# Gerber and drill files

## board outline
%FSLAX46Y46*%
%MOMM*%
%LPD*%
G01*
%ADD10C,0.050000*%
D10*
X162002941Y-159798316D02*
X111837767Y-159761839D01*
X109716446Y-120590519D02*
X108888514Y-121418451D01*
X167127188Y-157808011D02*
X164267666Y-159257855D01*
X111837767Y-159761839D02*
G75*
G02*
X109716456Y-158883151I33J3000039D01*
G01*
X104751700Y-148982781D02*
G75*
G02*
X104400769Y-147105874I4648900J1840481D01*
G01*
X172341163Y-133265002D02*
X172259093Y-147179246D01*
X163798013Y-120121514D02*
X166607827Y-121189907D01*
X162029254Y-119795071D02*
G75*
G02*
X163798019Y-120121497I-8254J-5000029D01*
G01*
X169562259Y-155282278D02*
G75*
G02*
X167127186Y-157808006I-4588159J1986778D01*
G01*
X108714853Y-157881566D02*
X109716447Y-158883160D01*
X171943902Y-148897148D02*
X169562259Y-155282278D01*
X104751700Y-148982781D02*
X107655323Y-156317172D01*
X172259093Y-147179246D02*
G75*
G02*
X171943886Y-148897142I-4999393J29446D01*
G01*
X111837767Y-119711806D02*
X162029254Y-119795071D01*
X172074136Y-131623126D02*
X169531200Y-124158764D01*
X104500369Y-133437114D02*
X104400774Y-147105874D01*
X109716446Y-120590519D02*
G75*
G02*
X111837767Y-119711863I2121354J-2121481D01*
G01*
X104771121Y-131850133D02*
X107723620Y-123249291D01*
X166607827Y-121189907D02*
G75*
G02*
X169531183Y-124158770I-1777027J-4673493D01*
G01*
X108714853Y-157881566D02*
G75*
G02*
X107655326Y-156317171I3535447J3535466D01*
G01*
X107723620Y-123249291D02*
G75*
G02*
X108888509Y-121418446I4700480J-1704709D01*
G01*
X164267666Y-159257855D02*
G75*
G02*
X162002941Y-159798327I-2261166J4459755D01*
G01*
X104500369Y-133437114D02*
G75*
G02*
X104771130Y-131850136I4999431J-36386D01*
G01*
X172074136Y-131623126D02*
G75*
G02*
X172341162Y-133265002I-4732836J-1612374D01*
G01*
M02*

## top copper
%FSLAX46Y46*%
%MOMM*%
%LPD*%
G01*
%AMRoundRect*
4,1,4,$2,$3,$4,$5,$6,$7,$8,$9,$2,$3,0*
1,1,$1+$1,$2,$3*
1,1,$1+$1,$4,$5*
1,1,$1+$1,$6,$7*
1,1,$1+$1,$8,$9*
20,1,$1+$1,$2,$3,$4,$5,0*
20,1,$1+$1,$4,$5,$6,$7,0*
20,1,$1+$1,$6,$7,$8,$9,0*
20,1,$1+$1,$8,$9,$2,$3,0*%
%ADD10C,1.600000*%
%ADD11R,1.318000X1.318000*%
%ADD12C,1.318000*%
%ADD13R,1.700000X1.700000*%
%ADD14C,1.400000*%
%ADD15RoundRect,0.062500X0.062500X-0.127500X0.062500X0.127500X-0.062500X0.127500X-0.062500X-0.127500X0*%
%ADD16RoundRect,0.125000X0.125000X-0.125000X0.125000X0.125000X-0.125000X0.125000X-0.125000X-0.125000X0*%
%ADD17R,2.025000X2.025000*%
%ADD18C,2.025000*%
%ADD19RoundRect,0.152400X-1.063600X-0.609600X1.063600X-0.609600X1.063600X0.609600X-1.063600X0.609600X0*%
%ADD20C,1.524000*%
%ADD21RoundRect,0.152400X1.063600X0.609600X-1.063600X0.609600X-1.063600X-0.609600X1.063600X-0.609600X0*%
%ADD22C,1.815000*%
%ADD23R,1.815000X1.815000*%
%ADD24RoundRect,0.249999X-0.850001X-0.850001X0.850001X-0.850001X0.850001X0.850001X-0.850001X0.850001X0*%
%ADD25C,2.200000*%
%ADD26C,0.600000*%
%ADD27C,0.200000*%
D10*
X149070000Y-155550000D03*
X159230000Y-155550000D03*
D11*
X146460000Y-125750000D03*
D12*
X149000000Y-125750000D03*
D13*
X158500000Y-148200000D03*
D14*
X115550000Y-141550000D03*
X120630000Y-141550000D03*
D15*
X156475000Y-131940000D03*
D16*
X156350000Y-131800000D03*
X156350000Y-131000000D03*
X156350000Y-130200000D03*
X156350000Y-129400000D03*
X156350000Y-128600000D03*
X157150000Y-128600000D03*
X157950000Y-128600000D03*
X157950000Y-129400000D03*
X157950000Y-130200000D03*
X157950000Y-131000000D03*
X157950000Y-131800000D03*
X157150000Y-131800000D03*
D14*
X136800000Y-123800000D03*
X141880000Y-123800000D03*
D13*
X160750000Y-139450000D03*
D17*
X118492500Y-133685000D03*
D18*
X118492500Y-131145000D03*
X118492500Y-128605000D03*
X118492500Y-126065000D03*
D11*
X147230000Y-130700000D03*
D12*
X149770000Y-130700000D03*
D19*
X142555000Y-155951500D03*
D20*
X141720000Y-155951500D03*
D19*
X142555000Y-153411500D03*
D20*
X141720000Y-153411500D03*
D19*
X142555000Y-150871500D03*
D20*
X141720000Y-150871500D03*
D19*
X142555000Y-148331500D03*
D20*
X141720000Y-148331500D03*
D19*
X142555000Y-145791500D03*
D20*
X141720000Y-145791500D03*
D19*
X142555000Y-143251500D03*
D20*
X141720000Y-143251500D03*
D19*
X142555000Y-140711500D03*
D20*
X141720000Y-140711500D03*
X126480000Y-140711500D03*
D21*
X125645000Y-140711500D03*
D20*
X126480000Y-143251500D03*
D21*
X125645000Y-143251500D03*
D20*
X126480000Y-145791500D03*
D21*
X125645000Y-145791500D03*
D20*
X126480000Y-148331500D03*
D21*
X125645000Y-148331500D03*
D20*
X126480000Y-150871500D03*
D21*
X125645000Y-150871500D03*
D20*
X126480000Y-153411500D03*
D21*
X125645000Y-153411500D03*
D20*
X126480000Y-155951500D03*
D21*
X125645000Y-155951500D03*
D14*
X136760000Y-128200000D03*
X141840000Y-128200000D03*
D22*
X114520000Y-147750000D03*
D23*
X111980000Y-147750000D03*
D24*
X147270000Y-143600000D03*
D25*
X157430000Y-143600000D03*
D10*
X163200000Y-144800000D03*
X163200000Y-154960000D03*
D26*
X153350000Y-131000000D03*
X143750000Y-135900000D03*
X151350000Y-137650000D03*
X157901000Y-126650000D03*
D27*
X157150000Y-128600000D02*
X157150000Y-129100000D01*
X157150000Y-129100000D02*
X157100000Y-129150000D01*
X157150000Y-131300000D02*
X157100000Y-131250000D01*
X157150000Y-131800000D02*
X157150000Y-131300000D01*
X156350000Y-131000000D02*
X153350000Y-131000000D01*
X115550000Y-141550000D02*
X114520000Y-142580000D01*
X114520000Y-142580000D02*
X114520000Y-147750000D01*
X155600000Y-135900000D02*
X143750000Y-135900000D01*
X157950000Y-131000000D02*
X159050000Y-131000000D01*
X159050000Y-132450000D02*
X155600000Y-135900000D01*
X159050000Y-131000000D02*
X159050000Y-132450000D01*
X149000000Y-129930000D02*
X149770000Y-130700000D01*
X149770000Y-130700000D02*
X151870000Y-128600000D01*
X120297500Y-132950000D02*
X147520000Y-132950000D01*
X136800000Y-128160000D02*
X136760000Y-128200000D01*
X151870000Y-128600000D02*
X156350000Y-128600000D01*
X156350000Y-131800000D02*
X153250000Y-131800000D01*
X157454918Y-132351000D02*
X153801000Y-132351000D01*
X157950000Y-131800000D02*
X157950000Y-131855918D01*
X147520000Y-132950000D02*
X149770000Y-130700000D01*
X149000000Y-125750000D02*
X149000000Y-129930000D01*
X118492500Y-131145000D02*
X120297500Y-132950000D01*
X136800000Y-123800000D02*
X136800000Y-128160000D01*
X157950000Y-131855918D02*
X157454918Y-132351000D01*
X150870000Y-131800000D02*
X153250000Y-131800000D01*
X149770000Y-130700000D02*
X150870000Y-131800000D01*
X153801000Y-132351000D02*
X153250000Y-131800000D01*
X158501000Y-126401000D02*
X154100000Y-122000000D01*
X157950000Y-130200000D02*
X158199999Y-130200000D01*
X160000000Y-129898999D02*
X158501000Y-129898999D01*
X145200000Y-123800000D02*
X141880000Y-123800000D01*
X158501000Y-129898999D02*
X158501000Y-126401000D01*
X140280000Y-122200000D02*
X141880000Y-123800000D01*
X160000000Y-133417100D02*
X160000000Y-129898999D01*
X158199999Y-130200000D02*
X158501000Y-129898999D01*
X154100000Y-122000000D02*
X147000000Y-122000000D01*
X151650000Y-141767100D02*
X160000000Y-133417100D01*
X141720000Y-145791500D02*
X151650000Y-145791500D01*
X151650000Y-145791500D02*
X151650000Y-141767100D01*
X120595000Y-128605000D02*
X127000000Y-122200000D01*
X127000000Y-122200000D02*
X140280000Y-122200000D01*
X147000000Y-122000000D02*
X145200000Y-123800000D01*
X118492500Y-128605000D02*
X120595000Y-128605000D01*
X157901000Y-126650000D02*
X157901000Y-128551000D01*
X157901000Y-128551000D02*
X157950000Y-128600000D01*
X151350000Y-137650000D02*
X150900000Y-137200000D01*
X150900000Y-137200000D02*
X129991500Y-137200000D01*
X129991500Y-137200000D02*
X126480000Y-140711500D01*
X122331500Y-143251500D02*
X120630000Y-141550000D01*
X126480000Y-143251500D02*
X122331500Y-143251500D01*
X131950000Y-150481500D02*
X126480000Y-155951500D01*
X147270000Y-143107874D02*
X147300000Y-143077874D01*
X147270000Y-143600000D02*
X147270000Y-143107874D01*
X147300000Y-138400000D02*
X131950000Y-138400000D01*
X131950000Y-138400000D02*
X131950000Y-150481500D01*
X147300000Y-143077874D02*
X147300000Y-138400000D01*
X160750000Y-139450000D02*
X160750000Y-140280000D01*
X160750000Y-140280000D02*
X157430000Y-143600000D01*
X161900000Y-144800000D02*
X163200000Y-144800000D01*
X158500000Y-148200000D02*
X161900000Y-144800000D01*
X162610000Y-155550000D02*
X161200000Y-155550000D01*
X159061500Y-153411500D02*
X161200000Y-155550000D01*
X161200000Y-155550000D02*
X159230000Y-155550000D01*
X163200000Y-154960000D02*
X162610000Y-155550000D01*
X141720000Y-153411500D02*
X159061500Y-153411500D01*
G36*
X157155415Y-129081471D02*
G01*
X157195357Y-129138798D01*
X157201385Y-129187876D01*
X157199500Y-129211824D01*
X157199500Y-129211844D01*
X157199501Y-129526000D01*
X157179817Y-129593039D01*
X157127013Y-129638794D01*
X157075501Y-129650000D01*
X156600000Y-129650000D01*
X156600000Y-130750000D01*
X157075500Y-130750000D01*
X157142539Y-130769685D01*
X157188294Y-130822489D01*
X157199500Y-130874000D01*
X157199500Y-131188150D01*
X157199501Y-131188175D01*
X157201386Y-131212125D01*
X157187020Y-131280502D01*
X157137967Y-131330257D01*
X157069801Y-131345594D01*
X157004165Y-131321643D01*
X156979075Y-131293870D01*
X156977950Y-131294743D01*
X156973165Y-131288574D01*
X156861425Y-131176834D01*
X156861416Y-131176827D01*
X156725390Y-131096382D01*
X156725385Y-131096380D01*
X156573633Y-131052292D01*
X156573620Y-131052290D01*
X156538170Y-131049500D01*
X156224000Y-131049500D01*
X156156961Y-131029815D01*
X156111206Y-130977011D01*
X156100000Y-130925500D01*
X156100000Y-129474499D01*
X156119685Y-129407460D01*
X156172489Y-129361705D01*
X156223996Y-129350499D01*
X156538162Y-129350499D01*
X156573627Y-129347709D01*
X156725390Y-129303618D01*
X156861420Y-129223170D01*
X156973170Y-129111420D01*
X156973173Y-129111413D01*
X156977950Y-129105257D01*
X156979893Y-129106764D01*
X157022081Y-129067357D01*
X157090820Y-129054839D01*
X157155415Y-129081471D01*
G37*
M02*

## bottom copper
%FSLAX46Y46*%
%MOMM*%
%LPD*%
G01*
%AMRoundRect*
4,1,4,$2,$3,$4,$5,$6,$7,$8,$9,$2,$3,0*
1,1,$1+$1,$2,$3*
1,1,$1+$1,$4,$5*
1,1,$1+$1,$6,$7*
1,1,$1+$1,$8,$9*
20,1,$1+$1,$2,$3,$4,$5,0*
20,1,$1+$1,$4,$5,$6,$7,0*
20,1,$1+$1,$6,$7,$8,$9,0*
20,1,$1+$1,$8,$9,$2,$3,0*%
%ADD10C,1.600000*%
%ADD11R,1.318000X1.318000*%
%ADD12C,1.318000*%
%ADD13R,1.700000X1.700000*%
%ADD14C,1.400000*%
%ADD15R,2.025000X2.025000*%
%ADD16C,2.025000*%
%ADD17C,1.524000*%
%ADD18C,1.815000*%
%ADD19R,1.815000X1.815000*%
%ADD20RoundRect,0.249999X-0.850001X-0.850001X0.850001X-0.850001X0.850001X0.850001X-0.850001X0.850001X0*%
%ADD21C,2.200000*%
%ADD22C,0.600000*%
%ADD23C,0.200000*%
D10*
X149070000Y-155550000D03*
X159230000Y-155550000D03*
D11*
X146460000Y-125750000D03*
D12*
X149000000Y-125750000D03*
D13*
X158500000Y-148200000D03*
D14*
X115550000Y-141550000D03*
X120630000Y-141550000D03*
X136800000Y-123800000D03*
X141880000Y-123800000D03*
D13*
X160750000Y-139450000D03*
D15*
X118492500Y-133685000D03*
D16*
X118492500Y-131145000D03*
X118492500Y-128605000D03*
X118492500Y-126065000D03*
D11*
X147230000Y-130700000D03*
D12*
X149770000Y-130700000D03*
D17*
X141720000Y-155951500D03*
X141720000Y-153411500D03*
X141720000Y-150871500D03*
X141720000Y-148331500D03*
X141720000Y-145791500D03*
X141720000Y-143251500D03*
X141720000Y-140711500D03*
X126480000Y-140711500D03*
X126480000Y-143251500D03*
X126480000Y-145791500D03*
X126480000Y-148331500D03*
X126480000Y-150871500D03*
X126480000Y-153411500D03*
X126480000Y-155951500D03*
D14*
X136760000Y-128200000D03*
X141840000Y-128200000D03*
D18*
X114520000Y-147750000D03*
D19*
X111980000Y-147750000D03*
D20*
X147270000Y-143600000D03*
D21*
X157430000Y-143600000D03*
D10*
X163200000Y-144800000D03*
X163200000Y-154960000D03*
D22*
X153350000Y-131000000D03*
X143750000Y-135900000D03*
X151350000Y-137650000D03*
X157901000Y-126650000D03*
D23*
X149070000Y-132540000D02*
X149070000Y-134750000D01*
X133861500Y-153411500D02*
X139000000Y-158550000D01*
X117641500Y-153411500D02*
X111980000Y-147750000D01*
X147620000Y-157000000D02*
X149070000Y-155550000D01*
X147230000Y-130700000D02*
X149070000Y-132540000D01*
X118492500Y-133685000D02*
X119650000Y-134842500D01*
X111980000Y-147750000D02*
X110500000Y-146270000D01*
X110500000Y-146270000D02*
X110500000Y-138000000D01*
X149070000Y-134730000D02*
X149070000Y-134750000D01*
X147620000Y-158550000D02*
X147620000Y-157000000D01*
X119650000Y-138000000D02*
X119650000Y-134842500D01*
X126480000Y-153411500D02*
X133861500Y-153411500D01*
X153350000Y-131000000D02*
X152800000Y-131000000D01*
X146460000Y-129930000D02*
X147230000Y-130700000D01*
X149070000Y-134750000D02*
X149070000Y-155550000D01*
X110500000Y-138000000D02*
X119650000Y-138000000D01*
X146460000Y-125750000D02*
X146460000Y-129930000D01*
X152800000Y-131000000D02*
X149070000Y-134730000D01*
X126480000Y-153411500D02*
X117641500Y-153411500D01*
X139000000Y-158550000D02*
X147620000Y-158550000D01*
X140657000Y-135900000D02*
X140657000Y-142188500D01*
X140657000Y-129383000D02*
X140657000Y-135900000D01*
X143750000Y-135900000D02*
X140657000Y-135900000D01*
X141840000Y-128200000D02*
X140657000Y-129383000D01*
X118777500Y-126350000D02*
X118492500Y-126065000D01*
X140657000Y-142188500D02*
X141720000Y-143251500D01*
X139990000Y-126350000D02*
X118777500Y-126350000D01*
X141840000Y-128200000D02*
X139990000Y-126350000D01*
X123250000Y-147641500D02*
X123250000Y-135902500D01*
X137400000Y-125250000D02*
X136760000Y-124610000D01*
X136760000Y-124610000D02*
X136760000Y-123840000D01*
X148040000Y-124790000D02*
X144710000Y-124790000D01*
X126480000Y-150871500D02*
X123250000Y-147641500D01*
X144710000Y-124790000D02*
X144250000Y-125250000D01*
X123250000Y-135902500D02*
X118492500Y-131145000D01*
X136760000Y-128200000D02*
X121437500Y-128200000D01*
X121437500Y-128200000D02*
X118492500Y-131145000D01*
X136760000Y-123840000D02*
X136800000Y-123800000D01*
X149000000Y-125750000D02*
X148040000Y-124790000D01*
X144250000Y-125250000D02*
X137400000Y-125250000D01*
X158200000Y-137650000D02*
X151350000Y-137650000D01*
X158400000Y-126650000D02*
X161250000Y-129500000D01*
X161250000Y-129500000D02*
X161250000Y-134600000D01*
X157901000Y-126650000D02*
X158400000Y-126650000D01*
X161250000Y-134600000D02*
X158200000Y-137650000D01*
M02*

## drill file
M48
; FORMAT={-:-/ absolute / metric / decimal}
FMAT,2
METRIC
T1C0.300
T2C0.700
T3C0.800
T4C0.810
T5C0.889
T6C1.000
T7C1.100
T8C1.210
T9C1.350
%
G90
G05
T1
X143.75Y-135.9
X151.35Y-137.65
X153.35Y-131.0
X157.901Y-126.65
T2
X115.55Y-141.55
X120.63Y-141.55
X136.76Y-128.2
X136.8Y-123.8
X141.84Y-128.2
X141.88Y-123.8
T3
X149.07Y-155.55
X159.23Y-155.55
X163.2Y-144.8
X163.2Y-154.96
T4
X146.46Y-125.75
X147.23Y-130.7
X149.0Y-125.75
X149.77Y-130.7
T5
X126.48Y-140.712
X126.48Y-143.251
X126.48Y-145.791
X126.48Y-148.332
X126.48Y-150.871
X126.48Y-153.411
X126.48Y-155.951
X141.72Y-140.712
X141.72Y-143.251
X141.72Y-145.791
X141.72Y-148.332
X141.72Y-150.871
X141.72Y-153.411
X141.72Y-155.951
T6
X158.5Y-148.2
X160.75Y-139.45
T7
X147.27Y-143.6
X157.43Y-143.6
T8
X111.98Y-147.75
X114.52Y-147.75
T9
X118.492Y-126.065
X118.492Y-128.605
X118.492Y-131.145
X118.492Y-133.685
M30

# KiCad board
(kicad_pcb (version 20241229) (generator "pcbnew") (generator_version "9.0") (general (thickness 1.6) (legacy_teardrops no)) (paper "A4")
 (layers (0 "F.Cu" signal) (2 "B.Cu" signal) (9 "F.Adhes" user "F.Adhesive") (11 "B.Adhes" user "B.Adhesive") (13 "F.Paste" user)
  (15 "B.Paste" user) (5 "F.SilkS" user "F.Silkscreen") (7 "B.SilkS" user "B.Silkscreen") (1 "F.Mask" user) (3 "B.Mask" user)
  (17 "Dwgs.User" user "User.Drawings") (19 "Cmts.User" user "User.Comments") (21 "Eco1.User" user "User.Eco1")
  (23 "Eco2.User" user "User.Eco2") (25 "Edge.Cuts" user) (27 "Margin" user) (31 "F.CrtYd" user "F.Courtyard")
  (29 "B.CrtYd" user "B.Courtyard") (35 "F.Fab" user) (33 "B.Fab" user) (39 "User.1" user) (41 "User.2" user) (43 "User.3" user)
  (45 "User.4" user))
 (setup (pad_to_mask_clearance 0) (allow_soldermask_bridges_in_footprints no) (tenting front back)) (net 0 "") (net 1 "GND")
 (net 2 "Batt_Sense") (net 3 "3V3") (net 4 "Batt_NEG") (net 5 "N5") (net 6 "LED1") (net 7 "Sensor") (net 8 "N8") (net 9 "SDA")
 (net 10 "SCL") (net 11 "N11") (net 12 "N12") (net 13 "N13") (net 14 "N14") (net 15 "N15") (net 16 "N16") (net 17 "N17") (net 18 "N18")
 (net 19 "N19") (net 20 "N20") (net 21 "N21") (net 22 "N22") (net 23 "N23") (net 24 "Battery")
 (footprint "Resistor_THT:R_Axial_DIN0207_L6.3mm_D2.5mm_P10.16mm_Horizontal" (layer "F.Cu") (at 149.07 155.55)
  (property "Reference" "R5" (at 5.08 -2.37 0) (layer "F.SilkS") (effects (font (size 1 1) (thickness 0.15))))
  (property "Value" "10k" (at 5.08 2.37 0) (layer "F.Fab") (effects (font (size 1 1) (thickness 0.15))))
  (pad "1" thru_hole circle (at 0 0) (size 1.6 1.6) (drill 0.8) (layers "*.Cu" "*.Mask") (remove_unused_layers no) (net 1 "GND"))
  (pad "2" thru_hole circle (at 10.16 0) (size 1.6 1.6) (drill 0.8) (layers "*.Cu" "*.Mask") (remove_unused_layers no) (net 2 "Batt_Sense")))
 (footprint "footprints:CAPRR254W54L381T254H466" (layer "F.Cu") (at 147.73 125.75)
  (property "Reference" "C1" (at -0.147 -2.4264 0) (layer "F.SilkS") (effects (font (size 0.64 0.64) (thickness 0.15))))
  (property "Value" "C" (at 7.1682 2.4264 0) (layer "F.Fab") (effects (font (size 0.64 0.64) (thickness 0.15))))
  (pad "1" thru_hole rect (at -1.27 0) (size 1.318 1.318) (drill 0.81) (layers "*.Cu" "*.Mask") (remove_unused_layers no) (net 1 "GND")
   (solder_mask_margin 0.102))
  (pad "2" thru_hole circle (at 1.27 0) (size 1.318 1.318) (drill 0.81) (layers "*.Cu" "*.Mask") (remove_unused_layers no) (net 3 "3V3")
   (solder_mask_margin 0.102)))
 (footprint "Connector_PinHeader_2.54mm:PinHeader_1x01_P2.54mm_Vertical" (layer "F.Cu") (at 158.5 148.2)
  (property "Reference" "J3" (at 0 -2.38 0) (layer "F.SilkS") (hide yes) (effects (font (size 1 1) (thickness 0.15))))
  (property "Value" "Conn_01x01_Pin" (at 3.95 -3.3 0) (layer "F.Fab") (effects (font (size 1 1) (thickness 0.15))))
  (pad "1" thru_hole rect (at 0 0) (size 1.7 1.7) (drill 1) (layers "*.Cu" "*.Mask") (remove_unused_layers no) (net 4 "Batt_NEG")))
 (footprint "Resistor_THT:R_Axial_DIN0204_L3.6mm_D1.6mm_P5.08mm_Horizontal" (layer "F.Cu") (at 115.55 141.55)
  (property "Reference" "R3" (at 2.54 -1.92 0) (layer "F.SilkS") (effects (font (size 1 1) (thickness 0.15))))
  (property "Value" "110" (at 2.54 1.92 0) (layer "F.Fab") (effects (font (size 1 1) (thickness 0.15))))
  (pad "1" thru_hole circle (at 0 0) (size 1.4 1.4) (drill 0.7) (layers "*.Cu" "*.Mask") (remove_unused_layers no) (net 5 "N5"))
  (pad "2" thru_hole circle (at 5.08 0) (size 1.4 1.4) (drill 0.7) (layers "*.Cu" "*.Mask") (remove_unused_layers no) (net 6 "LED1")))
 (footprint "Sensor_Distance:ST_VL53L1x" (layer "F.Cu") (at 157.15 130.2 90)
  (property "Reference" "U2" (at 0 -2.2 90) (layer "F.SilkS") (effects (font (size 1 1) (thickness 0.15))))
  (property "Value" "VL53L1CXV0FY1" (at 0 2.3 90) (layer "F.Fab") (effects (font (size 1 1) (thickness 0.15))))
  (pad "1" smd roundrect (at -1.74 -0.675 90) (size 0.38 0.25) (layers "F.Cu" "F.Mask" "F.Paste") (roundrect_rratio 0.25) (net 3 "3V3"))
  (pad "1" smd roundrect (at -1.6 -0.8 90) (size 0.5 0.5) (layers "F.Cu" "F.Mask" "F.Paste") (roundrect_rratio 0.25) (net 3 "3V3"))
  (pad "2" smd roundrect (at -0.8 -0.8 90) (size 0.5 0.5) (layers "F.Cu" "F.Mask" "F.Paste") (roundrect_rratio 0.25) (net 1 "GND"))
  (pad "3" smd roundrect (at 0 -0.8 90) (size 0.5 0.5) (layers "F.Cu" "F.Mask" "F.Paste") (roundrect_rratio 0.25) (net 1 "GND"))
  (pad "4" smd roundrect (at 0.8 -0.8 90) (size 0.5 0.5) (layers "F.Cu" "F.Mask" "F.Paste") (roundrect_rratio 0.25) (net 1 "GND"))
  (pad "5" smd roundrect (at 1.6 -0.8 90) (size 0.5 0.5) (layers "F.Cu" "F.Mask" "F.Paste") (roundrect_rratio 0.25) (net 3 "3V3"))
  (pad "6" smd roundrect (at 1.6 0 90) (size 0.5 0.5) (layers "F.Cu" "F.Mask" "F.Paste") (roundrect_rratio 0.25) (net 1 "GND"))
  (pad "7" smd roundrect (at 1.6 0.8 90) (size 0.5 0.5) (layers "F.Cu" "F.Mask" "F.Paste") (roundrect_rratio 0.25) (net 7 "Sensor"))
  (pad "8" smd roundrect (at 0.8 0.8 90) (size 0.5 0.5) (layers "F.Cu" "F.Mask" "F.Paste") (roundrect_rratio 0.25) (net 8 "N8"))
  (pad "9" smd roundrect (at 0 0.8 90) (size 0.5 0.5) (layers "F.Cu" "F.Mask" "F.Paste") (roundrect_rratio 0.25) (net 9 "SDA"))
  (pad "10" smd roundrect (at -0.8 0.8 90) (size 0.5 0.5) (layers "F.Cu" "F.Mask" "F.Paste") (roundrect_rratio 0.25) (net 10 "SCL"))
  (pad "11" smd roundrect (at -1.6 0.8 90) (size 0.5 0.5) (layers "F.Cu" "F.Mask" "F.Paste") (roundrect_rratio 0.25) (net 3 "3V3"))
  (pad "12" smd roundrect (at -1.6 0 90) (size 0.5 0.5) (layers "F.Cu" "F.Mask" "F.Paste") (roundrect_rratio 0.25) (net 1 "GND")))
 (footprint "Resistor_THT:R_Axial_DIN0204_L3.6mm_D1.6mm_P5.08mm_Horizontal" (layer "F.Cu") (at 136.8 123.8)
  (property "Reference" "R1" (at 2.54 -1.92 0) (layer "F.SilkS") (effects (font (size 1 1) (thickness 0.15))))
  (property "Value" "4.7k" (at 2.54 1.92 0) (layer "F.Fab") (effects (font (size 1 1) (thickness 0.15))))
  (pad "1" thru_hole circle (at 0 0) (size 1.4 1.4) (drill 0.7) (layers "*.Cu" "*.Mask") (remove_unused_layers no) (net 3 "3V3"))
  (pad "2" thru_hole circle (at 5.08 0) (size 1.4 1.4) (drill 0.7) (layers "*.Cu" "*.Mask") (remove_unused_layers no) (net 9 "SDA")))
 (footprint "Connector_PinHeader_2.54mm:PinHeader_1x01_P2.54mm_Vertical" (layer "F.Cu") (at 160.75 139.45)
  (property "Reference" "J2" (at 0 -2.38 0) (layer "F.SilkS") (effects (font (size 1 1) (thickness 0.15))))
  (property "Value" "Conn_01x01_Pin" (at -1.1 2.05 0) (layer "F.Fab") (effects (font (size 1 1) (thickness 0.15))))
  (pad "1" thru_hole rect (at 0 0) (size 1.7 1.7) (drill 1) (layers "*.Cu" "*.Mask") (remove_unused_layers no) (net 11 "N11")))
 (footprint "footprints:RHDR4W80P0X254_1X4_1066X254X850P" (layer "F.Cu") (at 118.4925 133.685 90)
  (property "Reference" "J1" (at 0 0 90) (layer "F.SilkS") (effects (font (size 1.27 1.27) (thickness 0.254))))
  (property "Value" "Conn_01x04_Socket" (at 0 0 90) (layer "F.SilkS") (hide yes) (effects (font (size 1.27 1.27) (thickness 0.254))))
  (pad "1" thru_hole rect (at 0 0 90) (size 2.025 2.025) (drill 1.35) (layers "*.Cu" "*.Mask") (remove_unused_layers no) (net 1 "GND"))
  (pad "2" thru_hole circle (at 2.54 0 90) (size 2.025 2.025) (drill 1.35) (layers "*.Cu" "*.Mask") (remove_unused_layers no) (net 3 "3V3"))
  (pad "3" thru_hole circle (at 5.08 0 90) (size 2.025 2.025) (drill 1.35) (layers "*.Cu" "*.Mask") (remove_unused_layers no) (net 9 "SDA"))
  (pad "4" thru_hole circle (at 7.62 0 90) (size 2.025 2.025) (drill 1.35) (layers "*.Cu" "*.Mask") (remove_unused_layers no) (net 10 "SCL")))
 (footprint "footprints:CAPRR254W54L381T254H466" (layer "F.Cu") (at 148.5 130.7)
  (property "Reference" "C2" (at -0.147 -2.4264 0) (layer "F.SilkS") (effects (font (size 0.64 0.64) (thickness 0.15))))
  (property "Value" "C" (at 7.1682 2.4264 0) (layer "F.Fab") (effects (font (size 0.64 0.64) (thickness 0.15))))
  (pad "1" thru_hole rect (at -1.27 0) (size 1.318 1.318) (drill 0.81) (layers "*.Cu" "*.Mask") (remove_unused_layers no) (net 1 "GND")
   (solder_mask_margin 0.102))
  (pad "2" thru_hole circle (at 1.27 0) (size 1.318 1.318) (drill 0.81) (layers "*.Cu" "*.Mask") (remove_unused_layers no) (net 3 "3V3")
   (solder_mask_margin 0.102)))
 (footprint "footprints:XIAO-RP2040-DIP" (layer "F.Cu") (at 134.1 148.3315 -90)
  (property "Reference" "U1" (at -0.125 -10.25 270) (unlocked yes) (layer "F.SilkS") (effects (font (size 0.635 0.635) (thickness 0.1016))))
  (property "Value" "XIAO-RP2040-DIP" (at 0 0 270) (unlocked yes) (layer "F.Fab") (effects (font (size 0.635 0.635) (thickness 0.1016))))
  (pad "1" smd roundrect (at 7.62 -8.455) (size 2.432 1.524) (layers "F.Cu" "F.Mask") (roundrect_rratio 0.1) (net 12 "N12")
   (thermal_bridge_angle 45))
  (pad "1" thru_hole circle (at 7.62 -7.62) (size 1.524 1.524) (drill 0.889) (layers "*.Cu" "*.Mask") (remove_unused_layers no)
   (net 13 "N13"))
  (pad "2" smd roundrect (at 5.08 -8.455) (size 2.432 1.524) (layers "F.Cu" "F.Mask") (roundrect_rratio 0.1) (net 2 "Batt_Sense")
   (thermal_bridge_angle 45))
  (pad "2" thru_hole circle (at 5.08 -7.62) (size 1.524 1.524) (drill 0.889) (layers "*.Cu" "*.Mask") (remove_unused_layers no)
   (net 2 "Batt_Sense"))
  (pad "3" smd roundrect (at 2.54 -8.455) (size 2.432 1.524) (layers "F.Cu" "F.Mask") (roundrect_rratio 0.1) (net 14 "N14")
   (thermal_bridge_angle 45))
  (pad "3" thru_hole circle (at 2.54 -7.62) (size 1.524 1.524) (drill 0.889) (layers "*.Cu" "*.Mask") (remove_unused_layers no)
   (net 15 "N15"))
  (pad "4" smd roundrect (at 0 -8.455) (size 2.432 1.524) (layers "F.Cu" "F.Mask") (roundrect_rratio 0.1) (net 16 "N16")
   (thermal_bridge_angle 45))
  (pad "4" thru_hole circle (at 0 -7.62) (size 1.524 1.524) (drill 0.889) (layers "*.Cu" "*.Mask") (remove_unused_layers no) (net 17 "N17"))
  (pad "5" smd roundrect (at -2.54 -8.455) (size 2.432 1.524) (layers "F.Cu" "F.Mask") (roundrect_rratio 0.1) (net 9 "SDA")
   (thermal_bridge_angle 45))
  (pad "5" thru_hole circle (at -2.54 -7.62) (size 1.524 1.524) (drill 0.889) (layers "*.Cu" "*.Mask") (remove_unused_layers no)
   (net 9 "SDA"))
  (pad "6" smd roundrect (at -5.08 -8.455) (size 2.432 1.524) (layers "F.Cu" "F.Mask") (roundrect_rratio 0.1) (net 10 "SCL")
   (thermal_bridge_angle 45))
  (pad "6" thru_hole circle (at -5.08 -7.62) (size 1.524 1.524) (drill 0.889) (layers "*.Cu" "*.Mask") (remove_unused_layers no)
   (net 10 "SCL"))
  (pad "7" smd roundrect (at -7.62 -8.455) (size 2.432 1.524) (layers "F.Cu" "F.Mask") (roundrect_rratio 0.1) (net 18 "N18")
   (thermal_bridge_angle 45))
  (pad "7" thru_hole circle (at -7.62 -7.62) (size 1.524 1.524) (drill 0.889) (layers "*.Cu" "*.Mask") (remove_unused_layers no)
   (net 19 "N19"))
  (pad "8" thru_hole circle (at -7.62 7.62 180) (size 1.524 1.524) (drill 0.889) (layers "*.Cu" "*.Mask") (remove_unused_layers no)
   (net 7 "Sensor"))
  (pad "8" smd roundrect (at -7.62 8.455 180) (size 2.432 1.524) (layers "F.Cu" "F.Mask") (roundrect_rratio 0.1) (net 7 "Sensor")
   (thermal_bridge_angle 45))
  (pad "9" thru_hole circle (at -5.08 7.62 180) (size 1.524 1.524) (drill 0.889) (layers "*.Cu" "*.Mask") (remove_unused_layers no)
   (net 6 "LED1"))
  (pad "9" smd roundrect (at -5.08 8.455 180) (size 2.432 1.524) (layers "F.Cu" "F.Mask") (roundrect_rratio 0.1) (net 6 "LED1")
   (thermal_bridge_angle 45))
  (pad "10" thru_hole circle (at -2.54 7.62 180) (size 1.524 1.524) (drill 0.889) (layers "*.Cu" "*.Mask") (remove_unused_layers no)
   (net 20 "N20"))
  (pad "10" smd roundrect (at -2.54 8.455 180) (size 2.432 1.524) (layers "F.Cu" "F.Mask") (roundrect_rratio 0.1) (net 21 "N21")
   (thermal_bridge_angle 45))
  (pad "11" thru_hole circle (at 0 7.62 180) (size 1.524 1.524) (drill 0.889) (layers "*.Cu" "*.Mask") (remove_unused_layers no)
   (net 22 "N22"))
  (pad "11" smd roundrect (at 0 8.455 180) (size 2.432 1.524) (layers "F.Cu" "F.Mask") (roundrect_rratio 0.1) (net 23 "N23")
   (thermal_bridge_angle 45))
  (pad "12" thru_hole circle (at 2.54 7.62 180) (size 1.524 1.524) (drill 0.889) (layers "*.Cu" "*.Mask") (remove_unused_layers no)
   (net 3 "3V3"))
  (pad "12" smd roundrect (at 2.54 8.455 180) (size 2.432 1.524) (layers "F.Cu" "F.Mask") (roundrect_rratio 0.1) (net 3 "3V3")
   (thermal_bridge_angle 45))
  (pad "13" thru_hole circle (at 5.08 7.62 180) (size 1.524 1.524) (drill 0.889) (layers "*.Cu" "*.Mask") (remove_unused_layers no)
   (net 1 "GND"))
  (pad "13" smd roundrect (at 5.08 8.455 180) (size 2.432 1.524) (layers "F.Cu" "F.Mask") (roundrect_rratio 0.1) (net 1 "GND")
   (thermal_bridge_angle 45))
  (pad "14" thru_hole circle (at 7.62 7.62 180) (size 1.524 1.524) (drill 0.889) (layers "*.Cu" "*.Mask") (remove_unused_layers no)
   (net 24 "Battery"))
  (pad "14" smd roundrect (at 7.62 8.455 180) (size 2.432 1.524) (layers "F.Cu" "F.Mask") (roundrect_rratio 0.1) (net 24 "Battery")
   (thermal_bridge_angle 45)))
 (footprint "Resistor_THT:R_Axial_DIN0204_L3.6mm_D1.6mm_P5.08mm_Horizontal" (layer "F.Cu") (at 136.76 128.2)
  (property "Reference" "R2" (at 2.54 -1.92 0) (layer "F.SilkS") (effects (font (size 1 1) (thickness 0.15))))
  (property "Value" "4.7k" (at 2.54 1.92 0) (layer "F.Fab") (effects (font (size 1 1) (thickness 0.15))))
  (pad "1" thru_hole circle (at 0 0) (size 1.4 1.4) (drill 0.7) (layers "*.Cu" "*.Mask") (remove_unused_layers no) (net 3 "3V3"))
  (pad "2" thru_hole circle (at 5.08 0) (size 1.4 1.4) (drill 0.7) (layers "*.Cu" "*.Mask") (remove_unused_layers no) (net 10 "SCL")))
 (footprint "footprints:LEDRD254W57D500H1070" (layer "F.Cu") (at 113.25 147.75)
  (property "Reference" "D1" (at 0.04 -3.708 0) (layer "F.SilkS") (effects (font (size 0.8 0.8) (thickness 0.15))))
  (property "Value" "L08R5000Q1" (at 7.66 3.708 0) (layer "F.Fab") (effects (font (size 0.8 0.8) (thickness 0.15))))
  (pad "A" thru_hole circle (at 1.27 0) (size 1.815 1.815) (drill 1.21) (layers "*.Cu" "*.Mask") (remove_unused_layers no) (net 5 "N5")
   (solder_mask_margin 0.102))
  (pad "C" thru_hole rect (at -1.27 0) (size 1.815 1.815) (drill 1.21) (layers "*.Cu" "*.Mask") (remove_unused_layers no) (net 1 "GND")
   (solder_mask_margin 0.102)))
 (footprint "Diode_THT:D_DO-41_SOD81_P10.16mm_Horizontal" (layer "F.Cu") (at 147.27 143.6)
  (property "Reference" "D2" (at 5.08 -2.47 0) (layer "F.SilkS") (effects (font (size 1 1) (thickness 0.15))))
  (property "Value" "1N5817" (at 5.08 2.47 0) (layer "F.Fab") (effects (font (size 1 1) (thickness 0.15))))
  (pad "1" thru_hole roundrect (at 0 0) (size 2.2 2.2) (drill 1.1) (layers "*.Cu" "*.Mask") (remove_unused_layers no)
   (roundrect_rratio 0.113636) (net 24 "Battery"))
  (pad "2" thru_hole circle (at 10.16 0) (size 2.2 2.2) (drill 1.1) (layers "*.Cu" "*.Mask") (remove_unused_layers no) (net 11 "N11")))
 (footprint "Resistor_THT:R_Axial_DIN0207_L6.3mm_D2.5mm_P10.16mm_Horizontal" (layer "F.Cu") (at 163.2 144.8 -90)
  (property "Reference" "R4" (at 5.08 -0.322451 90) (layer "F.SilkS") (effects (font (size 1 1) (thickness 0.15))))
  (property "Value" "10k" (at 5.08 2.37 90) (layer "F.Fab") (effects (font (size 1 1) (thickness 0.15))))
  (pad "1" thru_hole circle (at 0 0 270) (size 1.6 1.6) (drill 0.8) (layers "*.Cu" "*.Mask") (remove_unused_layers no) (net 4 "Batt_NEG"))
  (pad "2" thru_hole circle (at 10.16 0 270) (size 1.6 1.6) (drill 0.8) (layers "*.Cu" "*.Mask") (remove_unused_layers no)
   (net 2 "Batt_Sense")))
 (gr_line (start 162.002941 159.798316) (end 111.837767 159.761839) (stroke (width 0.05) (type default)) (layer "Edge.Cuts"))
 (gr_line (start 109.716446 120.590519) (end 108.888514 121.418451) (stroke (width 0.05) (type default)) (layer "Edge.Cuts"))
 (gr_line (start 167.127188 157.808011) (end 164.267666 159.257855) (stroke (width 0.05) (type default)) (layer "Edge.Cuts"))
 (gr_arc (start 111.837767 159.761839) (mid 110.689717 159.533478) (end 109.716447 158.88316) (stroke (width 0.05) (type default))
  (layer "Edge.Cuts"))
 (gr_arc (start 104.7517 148.982781) (mid 104.485809 148.061235) (end 104.400774 147.105874) (stroke (width 0.05) (type default))
  (layer "Edge.Cuts"))
 (gr_line (start 172.341163 133.265002) (end 172.259093 147.179246) (stroke (width 0.05) (type default)) (layer "Edge.Cuts"))
 (gr_line (start 163.798013 120.121514) (end 166.607827 121.189907) (stroke (width 0.05) (type default)) (layer "Edge.Cuts"))
 (gr_arc (start 162.029254 119.795071) (mid 162.928433 119.878105) (end 163.798013 120.121514) (stroke (width 0.05) (type default))
  (layer "Edge.Cuts"))
 (gr_arc (start 169.562259 155.282278) (mid 168.573532 156.765742) (end 167.127188 157.808011) (stroke (width 0.05) (type default))
  (layer "Edge.Cuts"))
 (gr_line (start 108.714853 157.881566) (end 109.716447 158.88316) (stroke (width 0.05) (type default)) (layer "Edge.Cuts"))
 (gr_line (start 171.943902 148.897148) (end 169.562259 155.282278) (stroke (width 0.05) (type default)) (layer "Edge.Cuts"))
 (gr_line (start 104.7517 148.982781) (end 107.655323 156.317172) (stroke (width 0.05) (type default)) (layer "Edge.Cuts"))
 (gr_arc (start 172.259093 147.179246) (mid 172.177097 148.052068) (end 171.943902 148.897148) (stroke (width 0.05) (type default))
  (layer "Edge.Cuts"))
 (gr_line (start 111.837767 119.711806) (end 162.029254 119.795071) (stroke (width 0.05) (type default)) (layer "Edge.Cuts"))
 (gr_line (start 172.074136 131.623126) (end 169.5312 124.158764) (stroke (width 0.05) (type default)) (layer "Edge.Cuts"))
 (gr_line (start 104.500369 133.437114) (end 104.400774 147.105874) (stroke (width 0.05) (type default)) (layer "Edge.Cuts"))
 (gr_arc (start 109.716446 120.590519) (mid 110.689719 119.940214) (end 111.837767 119.711839) (stroke (width 0.05) (type default))
  (layer "Edge.Cuts"))
 (gr_line (start 104.771121 131.850133) (end 107.72362 123.249291) (stroke (width 0.05) (type default)) (layer "Edge.Cuts"))
 (gr_arc (start 166.607827 121.189907) (mid 168.393495 122.35532) (end 169.5312 124.158764) (stroke (width 0.05) (type default))
  (layer "Edge.Cuts"))
 (gr_arc (start 108.714853 157.881566) (mid 108.110519 157.149873) (end 107.655323 156.317172) (stroke (width 0.05) (type default))
  (layer "Edge.Cuts"))
 (gr_arc (start 107.72362 123.249291) (mid 108.205546 122.269913) (end 108.888514 121.418451) (stroke (width 0.05) (type default))
  (layer "Edge.Cuts"))
 (gr_arc (start 164.267666 159.257855) (mid 163.1672 159.661741) (end 162.002941 159.798316) (stroke (width 0.05) (type default))
  (layer "Edge.Cuts"))
 (gr_arc (start 104.500369 133.437114) (mid 104.571447 132.632653) (end 104.771121 131.850133) (stroke (width 0.05) (type default))
  (layer "Edge.Cuts"))
 (gr_arc (start 172.074136 131.623126) (mid 172.276408 132.432881) (end 172.341163 133.265002) (stroke (width 0.05) (type default))
  (layer "Edge.Cuts"))
 (segment (start 157.15 128.6) (end 157.15 129.1) (width 0.2) (layer "F.Cu") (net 1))
 (segment (start 157.15 129.1) (end 157.1 129.15) (width 0.2) (layer "F.Cu") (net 1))
 (segment (start 157.15 131.3) (end 157.1 131.25) (width 0.2) (layer "F.Cu") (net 1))
 (segment (start 157.15 131.8) (end 157.15 131.3) (width 0.2) (layer "F.Cu") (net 1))
 (segment (start 156.35 131) (end 153.35 131) (width 0.2) (layer "F.Cu") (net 1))
 (via (at 153.35 131) (size 0.6) (drill 0.3) (layers "F.Cu" "B.Cu") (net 1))
 (segment (start 149.07 132.54) (end 149.07 134.75) (width 0.2) (layer "B.Cu") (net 1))
 (segment (start 133.8615 153.4115) (end 139 158.55) (width 0.2) (layer "B.Cu") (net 1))
 (segment (start 117.6415 153.4115) (end 111.98 147.75) (width 0.2) (layer "B.Cu") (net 1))
 (segment (start 147.62 157) (end 149.07 155.55) (width 0.2) (layer "B.Cu") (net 1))
 (segment (start 147.23 130.7) (end 149.07 132.54) (width 0.2) (layer "B.Cu") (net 1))
 (segment (start 118.4925 133.685) (end 119.65 134.8425) (width 0.2) (layer "B.Cu") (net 1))
 (segment (start 111.98 147.75) (end 110.5 146.27) (width 0.2) (layer "B.Cu") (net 1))
 (segment (start 110.5 146.27) (end 110.5 138) (width 0.2) (layer "B.Cu") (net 1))
 (segment (start 149.07 134.73) (end 149.07 134.75) (width 0.2) (layer "B.Cu") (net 1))
 (segment (start 147.62 158.55) (end 147.62 157) (width 0.2) (layer "B.Cu") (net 1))
 (segment (start 119.65 138) (end 119.65 134.8425) (width 0.2) (layer "B.Cu") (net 1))
 (segment (start 126.48 153.4115) (end 133.8615 153.4115) (width 0.2) (layer "B.Cu") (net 1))
 (segment (start 153.35 131) (end 152.8 131) (width 0.2) (layer "B.Cu") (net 1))
 (segment (start 146.46 129.93) (end 147.23 130.7) (width 0.2) (layer "B.Cu") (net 1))
 (segment (start 149.07 134.75) (end 149.07 155.55) (width 0.2) (layer "B.Cu") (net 1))
 (segment (start 110.5 138) (end 119.65 138) (width 0.2) (layer "B.Cu") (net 1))
 (segment (start 146.46 125.75) (end 146.46 129.93) (width 0.2) (layer "B.Cu") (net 1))
 (segment (start 152.8 131) (end 149.07 134.73) (width 0.2) (layer "B.Cu") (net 1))
 (segment (start 126.48 153.4115) (end 117.6415 153.4115) (width 0.2) (layer "B.Cu") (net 1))
 (segment (start 139 158.55) (end 147.62 158.55) (width 0.2) (layer "B.Cu") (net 1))
 (segment (start 115.55 141.55) (end 114.52 142.58) (width 0.2) (layer "F.Cu") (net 5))
 (segment (start 114.52 142.58) (end 114.52 147.75) (width 0.2) (layer "F.Cu") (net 5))
 (segment (start 155.6 135.9) (end 143.75 135.9) (width 0.2) (layer "F.Cu") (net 10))
 (segment (start 157.95 131) (end 159.05 131) (width 0.2) (layer "F.Cu") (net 10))
 (segment (start 159.05 132.45) (end 155.6 135.9) (width 0.2) (layer "F.Cu") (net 10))
 (segment (start 159.05 131) (end 159.05 132.45) (width 0.2) (layer "F.Cu") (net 10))
 (via (at 143.75 135.9) (size 0.6) (drill 0.3) (layers "F.Cu" "B.Cu") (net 10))
 (segment (start 140.657 135.9) (end 140.657 142.1885) (width 0.2) (layer "B.Cu") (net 10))
 (segment (start 140.657 129.383) (end 140.657 135.9) (width 0.2) (layer "B.Cu") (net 10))
 (segment (start 143.75 135.9) (end 140.657 135.9) (width 0.2) (layer "B.Cu") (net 10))
 (segment (start 141.84 128.2) (end 140.657 129.383) (width 0.2) (layer "B.Cu") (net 10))
 (segment (start 118.7775 126.35) (end 118.4925 126.065) (width 0.2) (layer "B.Cu") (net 10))
 (segment (start 140.657 142.1885) (end 141.72 143.2515) (width 0.2) (layer "B.Cu") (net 10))
 (segment (start 139.99 126.35) (end 118.7775 126.35) (width 0.2) (layer "B.Cu") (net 10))
 (segment (start 141.84 128.2) (end 139.99 126.35) (width 0.2) (layer "B.Cu") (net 10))
 (segment (start 149 129.93) (end 149.77 130.7) (width 0.2) (layer "F.Cu") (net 3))
 (segment (start 149.77 130.7) (end 151.87 128.6) (width 0.2) (layer "F.Cu") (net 3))
 (segment (start 120.2975 132.95) (end 147.52 132.95) (width 0.2) (layer "F.Cu") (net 3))
 (segment (start 136.8 128.16) (end 136.76 128.2) (width 0.2) (layer "F.Cu") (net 3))
 (segment (start 151.87 128.6) (end 156.35 128.6) (width 0.2) (layer "F.Cu") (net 3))
 (segment (start 156.35 131.8) (end 153.25 131.8) (width 0.2) (layer "F.Cu") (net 3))
 (segment (start 157.454918 132.351) (end 153.801 132.351) (width 0.2) (layer "F.Cu") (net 3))
 (segment (start 157.95 131.8) (end 157.95 131.855918) (width 0.2) (layer "F.Cu") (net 3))
 (segment (start 147.52 132.95) (end 149.77 130.7) (width 0.2) (layer "F.Cu") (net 3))
 (segment (start 149 125.75) (end 149 129.93) (width 0.2) (layer "F.Cu") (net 3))
 (segment (start 118.4925 131.145) (end 120.2975 132.95) (width 0.2) (layer "F.Cu") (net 3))
 (segment (start 136.8 123.8) (end 136.8 128.16) (width 0.2) (layer "F.Cu") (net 3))
 (segment (start 157.95 131.855918) (end 157.454918 132.351) (width 0.2) (layer "F.Cu") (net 3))
 (segment (start 150.87 131.8) (end 153.25 131.8) (width 0.2) (layer "F.Cu") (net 3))
 (segment (start 149.77 130.7) (end 150.87 131.8) (width 0.2) (layer "F.Cu") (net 3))
 (segment (start 153.801 132.351) (end 153.25 131.8) (width 0.2) (layer "F.Cu") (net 3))
 (segment (start 123.25 147.6415) (end 123.25 135.9025) (width 0.2) (layer "B.Cu") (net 3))
 (segment (start 137.4 125.25) (end 136.76 124.61) (width 0.2) (layer "B.Cu") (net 3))
 (segment (start 136.76 124.61) (end 136.76 123.84) (width 0.2) (layer "B.Cu") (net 3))
 (segment (start 148.04 124.79) (end 144.71 124.79) (width 0.2) (layer "B.Cu") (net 3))
 (segment (start 126.48 150.8715) (end 123.25 147.6415) (width 0.2) (layer "B.Cu") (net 3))
 (segment (start 144.71 124.79) (end 144.25 125.25) (width 0.2) (layer "B.Cu") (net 3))
 (segment (start 123.25 135.9025) (end 118.4925 131.145) (width 0.2) (layer "B.Cu") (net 3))
 (segment (start 136.76 128.2) (end 121.4375 128.2) (width 0.2) (layer "B.Cu") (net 3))
 (segment (start 121.4375 128.2) (end 118.4925 131.145) (width 0.2) (layer "B.Cu") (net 3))
 (segment (start 136.76 123.84) (end 136.8 123.8) (width 0.2) (layer "B.Cu") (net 3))
 (segment (start 149 125.75) (end 148.04 124.79) (width 0.2) (layer "B.Cu") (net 3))
 (segment (start 144.25 125.25) (end 137.4 125.25) (width 0.2) (layer "B.Cu") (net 3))
 (segment (start 158.501 126.401) (end 154.1 122) (width 0.2) (layer "F.Cu") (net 9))
 (segment (start 157.95 130.2) (end 158.199999 130.2) (width 0.2) (layer "F.Cu") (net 9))
 (segment (start 160 129.898999) (end 158.501 129.898999) (width 0.2) (layer "F.Cu") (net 9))
 (segment (start 145.2 123.8) (end 141.88 123.8) (width 0.2) (layer "F.Cu") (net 9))
 (segment (start 158.501 129.898999) (end 158.501 126.401) (width 0.2) (layer "F.Cu") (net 9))
 (segment (start 140.28 122.2) (end 141.88 123.8) (width 0.2) (layer "F.Cu") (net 9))
 (segment (start 160 133.4171) (end 160 129.898999) (width 0.2) (layer "F.Cu") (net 9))
 (segment (start 158.199999 130.2) (end 158.501 129.898999) (width 0.2) (layer "F.Cu") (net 9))
 (segment (start 154.1 122) (end 147 122) (width 0.2) (layer "F.Cu") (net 9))
 (segment (start 151.65 141.7671) (end 160 133.4171) (width 0.2) (layer "F.Cu") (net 9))
 (segment (start 141.72 145.7915) (end 151.65 145.7915) (width 0.2) (layer "F.Cu") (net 9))
 (segment (start 151.65 145.7915) (end 151.65 141.7671) (width 0.2) (layer "F.Cu") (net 9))
 (segment (start 120.595 128.605) (end 127 122.2) (width 0.2) (layer "F.Cu") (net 9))
 (segment (start 127 122.2) (end 140.28 122.2) (width 0.2) (layer "F.Cu") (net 9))
 (segment (start 147 122) (end 145.2 123.8) (width 0.2) (layer "F.Cu") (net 9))
 (segment (start 118.4925 128.605) (end 120.595 128.605) (width 0.2) (layer "F.Cu") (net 9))
 (segment (start 157.901 126.65) (end 157.901 128.551) (width 0.2) (layer "F.Cu") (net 7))
 (segment (start 157.901 128.551) (end 157.95 128.6) (width 0.2) (layer "F.Cu") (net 7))
 (segment (start 151.35 137.65) (end 150.9 137.2) (width 0.2) (layer "F.Cu") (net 7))
 (segment (start 150.9 137.2) (end 129.9915 137.2) (width 0.2) (layer "F.Cu") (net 7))
 (segment (start 129.9915 137.2) (end 126.48 140.7115) (width 0.2) (layer "F.Cu") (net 7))
 (via (at 151.35 137.65) (size 0.6) (drill 0.3) (layers "F.Cu" "B.Cu") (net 7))
 (via (at 157.901 126.65) (size 0.6) (drill 0.3) (layers "F.Cu" "B.Cu") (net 7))
 (segment (start 158.2 137.65) (end 151.35 137.65) (width 0.2) (layer "B.Cu") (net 7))
 (segment (start 158.4 126.65) (end 161.25 129.5) (width 0.2) (layer "B.Cu") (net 7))
 (segment (start 161.25 129.5) (end 161.25 134.6) (width 0.2) (layer "B.Cu") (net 7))
 (segment (start 157.901 126.65) (end 158.4 126.65) (width 0.2) (layer "B.Cu") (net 7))
 (segment (start 161.25 134.6) (end 158.2 137.65) (width 0.2) (layer "B.Cu") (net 7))
 (segment (start 122.3315 143.2515) (end 120.63 141.55) (width 0.2) (layer "F.Cu") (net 6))
 (segment (start 126.48 143.2515) (end 122.3315 143.2515) (width 0.2) (layer "F.Cu") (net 6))
 (segment (start 131.95 150.4815) (end 126.48 155.9515) (width 0.2) (layer "F.Cu") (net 24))
 (segment (start 147.27 143.107874) (end 147.3 143.077874) (width 0.2) (layer "F.Cu") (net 24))
 (segment (start 147.27 143.6) (end 147.27 143.107874) (width 0.2) (layer "F.Cu") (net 24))
 (segment (start 147.3 138.4) (end 131.95 138.4) (width 0.2) (layer "F.Cu") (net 24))
 (segment (start 131.95 138.4) (end 131.95 150.4815) (width 0.2) (layer "F.Cu") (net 24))
 (segment (start 147.3 143.077874) (end 147.3 138.4) (width 0.2) (layer "F.Cu") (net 24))
 (segment (start 160.75 139.45) (end 160.75 140.28) (width 0.2) (layer "F.Cu") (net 11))
 (segment (start 160.75 140.28) (end 157.43 143.6) (width 0.2) (layer "F.Cu") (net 11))
 (segment (start 161.9 144.8) (end 163.2 144.8) (width 0.2) (layer "F.Cu") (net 4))
 (segment (start 158.5 148.2) (end 161.9 144.8) (width 0.2) (layer "F.Cu") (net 4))
 (segment (start 162.61 155.55) (end 161.2 155.55) (width 0.2) (layer "F.Cu") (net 2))
 (segment (start 159.0615 153.4115) (end 161.2 155.55) (width 0.2) (layer "F.Cu") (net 2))
 (segment (start 161.2 155.55) (end 159.23 155.55) (width 0.2) (layer "F.Cu") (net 2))
 (segment (start 163.2 154.96) (end 162.61 155.55) (width 0.2) (layer "F.Cu") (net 2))
 (segment (start 141.72 153.4115) (end 159.0615 153.4115) (width 0.2) (layer "F.Cu") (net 2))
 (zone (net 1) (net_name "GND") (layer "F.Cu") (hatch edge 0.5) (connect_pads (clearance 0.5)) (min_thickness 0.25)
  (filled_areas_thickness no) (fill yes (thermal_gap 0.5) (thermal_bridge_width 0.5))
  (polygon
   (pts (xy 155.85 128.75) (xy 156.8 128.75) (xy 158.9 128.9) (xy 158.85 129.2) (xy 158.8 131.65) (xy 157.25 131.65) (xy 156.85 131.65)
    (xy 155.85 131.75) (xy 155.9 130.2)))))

